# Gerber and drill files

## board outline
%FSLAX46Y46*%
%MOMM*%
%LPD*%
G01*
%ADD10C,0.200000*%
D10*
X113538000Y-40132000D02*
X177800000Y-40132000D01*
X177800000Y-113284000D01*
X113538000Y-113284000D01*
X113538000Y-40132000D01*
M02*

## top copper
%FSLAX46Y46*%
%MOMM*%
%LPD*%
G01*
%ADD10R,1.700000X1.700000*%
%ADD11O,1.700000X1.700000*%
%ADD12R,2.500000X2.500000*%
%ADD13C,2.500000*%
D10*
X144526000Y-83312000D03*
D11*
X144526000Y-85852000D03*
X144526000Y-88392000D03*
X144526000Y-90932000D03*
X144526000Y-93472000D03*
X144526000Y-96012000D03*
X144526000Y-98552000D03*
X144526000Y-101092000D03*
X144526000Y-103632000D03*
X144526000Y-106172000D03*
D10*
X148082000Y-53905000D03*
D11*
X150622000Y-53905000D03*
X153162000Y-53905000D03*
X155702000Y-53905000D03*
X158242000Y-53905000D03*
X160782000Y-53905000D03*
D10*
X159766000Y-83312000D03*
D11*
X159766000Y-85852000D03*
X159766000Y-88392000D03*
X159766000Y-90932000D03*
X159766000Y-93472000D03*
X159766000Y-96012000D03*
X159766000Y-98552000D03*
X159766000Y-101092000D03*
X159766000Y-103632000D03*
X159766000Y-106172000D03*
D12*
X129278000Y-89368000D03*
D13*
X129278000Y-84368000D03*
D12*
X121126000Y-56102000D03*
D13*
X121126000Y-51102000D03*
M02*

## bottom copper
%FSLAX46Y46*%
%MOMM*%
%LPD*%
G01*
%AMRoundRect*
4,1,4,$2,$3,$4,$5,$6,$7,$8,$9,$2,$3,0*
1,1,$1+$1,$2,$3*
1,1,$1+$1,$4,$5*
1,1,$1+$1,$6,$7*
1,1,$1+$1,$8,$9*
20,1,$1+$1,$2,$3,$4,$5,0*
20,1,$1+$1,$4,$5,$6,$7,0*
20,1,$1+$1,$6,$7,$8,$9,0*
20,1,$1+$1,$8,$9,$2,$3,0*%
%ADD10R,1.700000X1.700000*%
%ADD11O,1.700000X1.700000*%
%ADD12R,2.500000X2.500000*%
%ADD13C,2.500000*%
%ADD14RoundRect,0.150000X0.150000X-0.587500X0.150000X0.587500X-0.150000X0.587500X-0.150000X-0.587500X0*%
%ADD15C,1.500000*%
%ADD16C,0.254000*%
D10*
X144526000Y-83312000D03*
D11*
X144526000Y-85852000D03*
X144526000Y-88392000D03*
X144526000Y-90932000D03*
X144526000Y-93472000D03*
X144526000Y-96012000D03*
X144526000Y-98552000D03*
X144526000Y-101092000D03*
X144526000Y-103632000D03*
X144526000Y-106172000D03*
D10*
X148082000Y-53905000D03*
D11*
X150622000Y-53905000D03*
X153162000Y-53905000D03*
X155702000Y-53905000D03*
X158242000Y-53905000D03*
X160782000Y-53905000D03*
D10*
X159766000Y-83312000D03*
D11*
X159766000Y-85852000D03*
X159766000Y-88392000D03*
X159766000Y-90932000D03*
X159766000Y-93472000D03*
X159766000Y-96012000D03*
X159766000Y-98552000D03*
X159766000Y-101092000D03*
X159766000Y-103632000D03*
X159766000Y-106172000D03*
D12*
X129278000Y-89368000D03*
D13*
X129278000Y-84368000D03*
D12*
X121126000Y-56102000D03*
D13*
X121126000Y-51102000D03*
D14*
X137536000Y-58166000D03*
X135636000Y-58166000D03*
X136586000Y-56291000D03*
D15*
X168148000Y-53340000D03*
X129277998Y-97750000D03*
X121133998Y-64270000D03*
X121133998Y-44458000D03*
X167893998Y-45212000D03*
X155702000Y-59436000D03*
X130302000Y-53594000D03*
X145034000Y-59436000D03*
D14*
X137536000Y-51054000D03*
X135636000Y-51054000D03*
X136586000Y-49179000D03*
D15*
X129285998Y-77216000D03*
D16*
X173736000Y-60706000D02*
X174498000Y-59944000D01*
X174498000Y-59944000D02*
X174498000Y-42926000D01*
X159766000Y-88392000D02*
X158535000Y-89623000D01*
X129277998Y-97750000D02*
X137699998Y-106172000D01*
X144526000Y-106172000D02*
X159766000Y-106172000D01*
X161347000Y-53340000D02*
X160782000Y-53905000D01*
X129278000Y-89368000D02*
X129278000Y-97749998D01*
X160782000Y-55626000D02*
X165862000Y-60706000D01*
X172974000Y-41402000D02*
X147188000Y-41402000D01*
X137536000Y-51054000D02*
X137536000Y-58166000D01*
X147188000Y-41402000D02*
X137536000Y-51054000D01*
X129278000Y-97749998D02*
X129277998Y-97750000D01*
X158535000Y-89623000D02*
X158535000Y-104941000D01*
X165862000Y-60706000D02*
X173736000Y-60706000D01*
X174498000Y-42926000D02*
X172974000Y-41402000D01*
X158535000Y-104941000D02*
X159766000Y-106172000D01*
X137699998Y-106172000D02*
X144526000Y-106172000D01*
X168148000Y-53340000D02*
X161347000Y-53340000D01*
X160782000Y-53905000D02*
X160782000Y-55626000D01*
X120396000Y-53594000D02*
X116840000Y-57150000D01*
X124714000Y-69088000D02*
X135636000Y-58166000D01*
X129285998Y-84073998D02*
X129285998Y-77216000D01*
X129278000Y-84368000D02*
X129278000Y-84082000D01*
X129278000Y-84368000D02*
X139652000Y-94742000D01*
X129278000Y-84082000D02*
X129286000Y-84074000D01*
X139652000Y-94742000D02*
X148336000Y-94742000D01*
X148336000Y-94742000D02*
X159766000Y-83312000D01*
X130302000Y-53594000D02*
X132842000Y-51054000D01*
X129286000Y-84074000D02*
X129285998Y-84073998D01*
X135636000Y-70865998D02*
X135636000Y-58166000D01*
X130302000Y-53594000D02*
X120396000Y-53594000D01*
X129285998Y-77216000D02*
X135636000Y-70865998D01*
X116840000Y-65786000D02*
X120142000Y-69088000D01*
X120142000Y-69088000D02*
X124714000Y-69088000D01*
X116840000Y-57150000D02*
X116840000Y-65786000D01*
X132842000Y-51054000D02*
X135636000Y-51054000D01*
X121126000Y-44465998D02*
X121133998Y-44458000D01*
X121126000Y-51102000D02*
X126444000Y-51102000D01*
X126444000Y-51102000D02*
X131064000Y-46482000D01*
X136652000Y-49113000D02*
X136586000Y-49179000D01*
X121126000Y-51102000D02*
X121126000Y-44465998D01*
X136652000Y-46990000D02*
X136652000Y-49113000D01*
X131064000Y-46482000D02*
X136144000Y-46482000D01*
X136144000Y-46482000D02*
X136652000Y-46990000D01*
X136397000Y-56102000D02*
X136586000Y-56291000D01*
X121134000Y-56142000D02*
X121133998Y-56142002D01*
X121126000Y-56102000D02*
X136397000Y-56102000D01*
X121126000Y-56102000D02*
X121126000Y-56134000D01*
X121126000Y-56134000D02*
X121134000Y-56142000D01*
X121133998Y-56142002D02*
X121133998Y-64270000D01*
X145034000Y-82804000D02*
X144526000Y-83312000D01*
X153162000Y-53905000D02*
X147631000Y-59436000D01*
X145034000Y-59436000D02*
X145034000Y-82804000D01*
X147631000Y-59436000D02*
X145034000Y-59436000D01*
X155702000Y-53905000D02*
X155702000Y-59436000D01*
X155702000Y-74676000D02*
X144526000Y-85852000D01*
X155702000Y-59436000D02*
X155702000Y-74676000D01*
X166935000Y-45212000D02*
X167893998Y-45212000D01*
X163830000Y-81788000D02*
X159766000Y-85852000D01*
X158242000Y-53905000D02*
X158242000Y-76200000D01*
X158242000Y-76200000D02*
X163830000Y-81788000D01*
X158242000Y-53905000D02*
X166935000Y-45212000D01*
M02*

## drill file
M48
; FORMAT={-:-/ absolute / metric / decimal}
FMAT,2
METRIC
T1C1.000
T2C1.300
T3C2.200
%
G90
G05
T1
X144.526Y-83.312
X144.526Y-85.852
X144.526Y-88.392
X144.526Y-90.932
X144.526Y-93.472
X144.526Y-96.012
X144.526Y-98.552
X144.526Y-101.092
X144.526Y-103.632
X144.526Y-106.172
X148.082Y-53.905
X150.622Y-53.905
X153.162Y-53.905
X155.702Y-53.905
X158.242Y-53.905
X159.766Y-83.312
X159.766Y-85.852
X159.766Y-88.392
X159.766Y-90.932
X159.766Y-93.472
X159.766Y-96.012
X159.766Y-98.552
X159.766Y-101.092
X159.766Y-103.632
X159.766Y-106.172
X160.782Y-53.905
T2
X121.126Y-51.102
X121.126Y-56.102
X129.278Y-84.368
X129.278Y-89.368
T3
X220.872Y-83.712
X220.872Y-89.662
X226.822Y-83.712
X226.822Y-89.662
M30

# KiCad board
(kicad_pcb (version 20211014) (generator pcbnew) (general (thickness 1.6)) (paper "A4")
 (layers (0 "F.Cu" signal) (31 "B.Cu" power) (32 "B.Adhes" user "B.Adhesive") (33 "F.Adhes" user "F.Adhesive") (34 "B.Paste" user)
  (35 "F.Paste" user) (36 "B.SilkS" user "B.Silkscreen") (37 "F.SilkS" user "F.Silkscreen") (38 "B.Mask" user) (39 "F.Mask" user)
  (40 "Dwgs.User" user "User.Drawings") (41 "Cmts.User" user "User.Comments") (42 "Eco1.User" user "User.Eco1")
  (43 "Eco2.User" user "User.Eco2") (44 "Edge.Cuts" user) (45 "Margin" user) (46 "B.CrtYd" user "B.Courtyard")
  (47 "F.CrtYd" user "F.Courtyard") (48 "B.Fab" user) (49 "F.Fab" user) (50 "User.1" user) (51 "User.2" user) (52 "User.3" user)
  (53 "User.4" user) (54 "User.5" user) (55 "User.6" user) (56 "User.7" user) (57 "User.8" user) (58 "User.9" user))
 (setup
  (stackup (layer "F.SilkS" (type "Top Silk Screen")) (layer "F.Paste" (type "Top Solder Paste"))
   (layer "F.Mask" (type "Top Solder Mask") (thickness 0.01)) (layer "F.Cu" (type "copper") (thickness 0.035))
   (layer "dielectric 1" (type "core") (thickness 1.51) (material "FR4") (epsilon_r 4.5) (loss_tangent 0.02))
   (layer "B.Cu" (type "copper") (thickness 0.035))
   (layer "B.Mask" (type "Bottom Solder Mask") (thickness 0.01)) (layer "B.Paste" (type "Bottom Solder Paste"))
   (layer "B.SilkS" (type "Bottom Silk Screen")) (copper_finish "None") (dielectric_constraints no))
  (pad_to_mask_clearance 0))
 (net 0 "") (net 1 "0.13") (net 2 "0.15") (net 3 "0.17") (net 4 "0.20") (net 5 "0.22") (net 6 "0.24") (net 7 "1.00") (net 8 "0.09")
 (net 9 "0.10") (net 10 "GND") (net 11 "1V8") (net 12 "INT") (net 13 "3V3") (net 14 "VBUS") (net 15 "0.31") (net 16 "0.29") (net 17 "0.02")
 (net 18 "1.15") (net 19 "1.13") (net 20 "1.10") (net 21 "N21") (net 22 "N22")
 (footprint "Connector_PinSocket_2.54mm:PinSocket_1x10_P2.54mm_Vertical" (layer "F.Cu") (at 144.526 83.312)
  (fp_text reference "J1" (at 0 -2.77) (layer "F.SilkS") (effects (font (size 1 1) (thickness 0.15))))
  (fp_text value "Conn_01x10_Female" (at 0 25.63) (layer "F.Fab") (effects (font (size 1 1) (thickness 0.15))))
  (pad "1" thru_hole rect (at 0 0) (size 1.7 1.7) (drill 1) (layers *.Cu *.Mask) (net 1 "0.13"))
  (pad "2" thru_hole oval (at 0 2.54) (size 1.7 1.7) (drill 1) (layers *.Cu *.Mask) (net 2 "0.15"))
  (pad "3" thru_hole oval (at 0 5.08) (size 1.7 1.7) (drill 1) (layers *.Cu *.Mask) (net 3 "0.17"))
  (pad "4" thru_hole oval (at 0 7.62) (size 1.7 1.7) (drill 1) (layers *.Cu *.Mask) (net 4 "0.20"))
  (pad "5" thru_hole oval (at 0 10.16) (size 1.7 1.7) (drill 1) (layers *.Cu *.Mask) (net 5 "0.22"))
  (pad "6" thru_hole oval (at 0 12.7) (size 1.7 1.7) (drill 1) (layers *.Cu *.Mask) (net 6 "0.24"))
  (pad "7" thru_hole oval (at 0 15.24) (size 1.7 1.7) (drill 1) (layers *.Cu *.Mask) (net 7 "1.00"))
  (pad "8" thru_hole oval (at 0 17.78) (size 1.7 1.7) (drill 1) (layers *.Cu *.Mask) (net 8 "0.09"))
  (pad "9" thru_hole oval (at 0 20.32) (size 1.7 1.7) (drill 1) (layers *.Cu *.Mask) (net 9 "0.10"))
  (pad "10" thru_hole oval (at 0 22.86) (size 1.7 1.7) (drill 1) (layers *.Cu *.Mask) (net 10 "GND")))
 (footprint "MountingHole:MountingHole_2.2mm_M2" (layer "F.Cu") (at 226.822 83.712)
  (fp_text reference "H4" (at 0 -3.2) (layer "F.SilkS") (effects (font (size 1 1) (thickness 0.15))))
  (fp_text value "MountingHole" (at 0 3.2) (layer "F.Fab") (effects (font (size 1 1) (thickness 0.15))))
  (pad "" np_thru_hole circle (at 0 0) (size 2.2 2.2) (drill 2.2) (layers *.Cu *.Mask)))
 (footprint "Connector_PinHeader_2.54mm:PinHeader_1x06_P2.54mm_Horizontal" (layer "F.Cu") (at 148.082 53.905 90)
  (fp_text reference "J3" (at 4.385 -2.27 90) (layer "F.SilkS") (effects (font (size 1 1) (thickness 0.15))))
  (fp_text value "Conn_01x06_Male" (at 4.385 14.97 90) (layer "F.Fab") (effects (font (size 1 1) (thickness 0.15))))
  (pad "1" thru_hole rect (at 0 0 90) (size 1.7 1.7) (drill 1) (layers *.Cu *.Mask) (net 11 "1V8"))
  (pad "2" thru_hole oval (at 0 2.54 90) (size 1.7 1.7) (drill 1) (layers *.Cu *.Mask) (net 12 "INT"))
  (pad "3" thru_hole oval (at 0 5.08 90) (size 1.7 1.7) (drill 1) (layers *.Cu *.Mask) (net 1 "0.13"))
  (pad "4" thru_hole oval (at 0 7.62 90) (size 1.7 1.7) (drill 1) (layers *.Cu *.Mask) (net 2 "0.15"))
  (pad "5" thru_hole oval (at 0 10.16 90) (size 1.7 1.7) (drill 1) (layers *.Cu *.Mask) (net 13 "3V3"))
  (pad "6" thru_hole oval (at 0 12.7 90) (size 1.7 1.7) (drill 1) (layers *.Cu *.Mask) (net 10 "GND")))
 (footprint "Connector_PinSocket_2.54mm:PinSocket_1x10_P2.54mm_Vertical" (layer "F.Cu") (at 159.766 83.312)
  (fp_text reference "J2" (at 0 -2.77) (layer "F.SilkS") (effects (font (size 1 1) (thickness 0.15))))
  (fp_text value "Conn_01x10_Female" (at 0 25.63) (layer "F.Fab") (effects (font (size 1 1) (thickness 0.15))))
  (pad "1" thru_hole rect (at 0 0) (size 1.7 1.7) (drill 1) (layers *.Cu *.Mask) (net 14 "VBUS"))
  (pad "2" thru_hole oval (at 0 2.54) (size 1.7 1.7) (drill 1) (layers *.Cu *.Mask) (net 13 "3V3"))
  (pad "3" thru_hole oval (at 0 5.08) (size 1.7 1.7) (drill 1) (layers *.Cu *.Mask) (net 10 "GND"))
  (pad "4" thru_hole oval (at 0 7.62) (size 1.7 1.7) (drill 1) (layers *.Cu *.Mask) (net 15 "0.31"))
  (pad "5" thru_hole oval (at 0 10.16) (size 1.7 1.7) (drill 1) (layers *.Cu *.Mask) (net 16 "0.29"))
  (pad "6" thru_hole oval (at 0 12.7) (size 1.7 1.7) (drill 1) (layers *.Cu *.Mask) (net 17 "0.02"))
  (pad "7" thru_hole oval (at 0 15.24) (size 1.7 1.7) (drill 1) (layers *.Cu *.Mask) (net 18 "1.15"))
  (pad "8" thru_hole oval (at 0 17.78) (size 1.7 1.7) (drill 1) (layers *.Cu *.Mask) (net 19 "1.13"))
  (pad "9" thru_hole oval (at 0 20.32) (size 1.7 1.7) (drill 1) (layers *.Cu *.Mask) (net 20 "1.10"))
  (pad "10" thru_hole oval (at 0 22.86) (size 1.7 1.7) (drill 1) (layers *.Cu *.Mask) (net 10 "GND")))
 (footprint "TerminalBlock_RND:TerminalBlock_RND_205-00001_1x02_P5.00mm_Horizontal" (layer "F.Cu") (at 129.278 89.368 90)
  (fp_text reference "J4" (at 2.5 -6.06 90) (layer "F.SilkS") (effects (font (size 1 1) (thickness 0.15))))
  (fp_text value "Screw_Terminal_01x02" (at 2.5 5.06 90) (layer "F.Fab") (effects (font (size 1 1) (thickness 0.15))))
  (pad "1" thru_hole rect (at 0 0 90) (size 2.5 2.5) (drill 1.3) (layers *.Cu *.Mask) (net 10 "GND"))
  (pad "2" thru_hole circle (at 5 0 90) (size 2.5 2.5) (drill 1.3) (layers *.Cu *.Mask) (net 14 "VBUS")))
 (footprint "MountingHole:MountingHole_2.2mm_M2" (layer "F.Cu") (at 226.822 89.662)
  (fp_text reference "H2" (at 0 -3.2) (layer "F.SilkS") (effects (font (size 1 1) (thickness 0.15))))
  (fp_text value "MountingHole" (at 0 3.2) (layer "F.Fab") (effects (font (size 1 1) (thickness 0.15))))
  (pad "" np_thru_hole circle (at 0 0) (size 2.2 2.2) (drill 2.2) (layers *.Cu *.Mask)))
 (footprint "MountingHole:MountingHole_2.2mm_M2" (layer "F.Cu") (at 220.872 89.662)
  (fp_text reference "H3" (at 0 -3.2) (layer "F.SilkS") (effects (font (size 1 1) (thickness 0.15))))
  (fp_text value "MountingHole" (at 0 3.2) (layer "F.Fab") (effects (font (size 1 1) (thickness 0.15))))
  (pad "" np_thru_hole circle (at 0 0) (size 2.2 2.2) (drill 2.2) (layers *.Cu *.Mask)))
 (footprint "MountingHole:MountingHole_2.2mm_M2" (layer "F.Cu") (at 220.872 83.712)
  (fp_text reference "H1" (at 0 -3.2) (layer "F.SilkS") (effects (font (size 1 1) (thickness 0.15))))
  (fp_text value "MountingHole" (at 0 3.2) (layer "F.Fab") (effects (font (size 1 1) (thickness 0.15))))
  (pad "" np_thru_hole circle (at 0 0) (size 2.2 2.2) (drill 2.2) (layers *.Cu *.Mask)))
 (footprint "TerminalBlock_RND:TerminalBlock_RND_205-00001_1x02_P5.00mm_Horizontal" (layer "F.Cu") (at 121.126 56.102 90)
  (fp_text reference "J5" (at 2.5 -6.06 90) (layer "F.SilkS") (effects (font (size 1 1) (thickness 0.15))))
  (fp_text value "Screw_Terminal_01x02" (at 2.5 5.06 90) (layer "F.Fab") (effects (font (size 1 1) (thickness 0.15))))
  (pad "1" thru_hole rect (at 0 0 90) (size 2.5 2.5) (drill 1.3) (layers *.Cu *.Mask) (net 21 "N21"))
  (pad "2" thru_hole circle (at 5 0 90) (size 2.5 2.5) (drill 1.3) (layers *.Cu *.Mask) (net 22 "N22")))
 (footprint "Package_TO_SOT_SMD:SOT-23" (layer "B.Cu") (at 136.586 57.2285 90)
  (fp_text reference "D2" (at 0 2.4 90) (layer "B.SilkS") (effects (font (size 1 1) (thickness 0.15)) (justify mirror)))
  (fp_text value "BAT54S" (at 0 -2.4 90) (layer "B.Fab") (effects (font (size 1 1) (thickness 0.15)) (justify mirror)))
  (pad "1" smd roundrect (at -0.9375 0.95 90) (size 1.475 0.6) (layers "B.Cu" "B.Paste" "B.Mask") (roundrect_rratio 0.25) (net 10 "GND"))
  (pad "2" smd roundrect (at -0.9375 -0.95 90) (size 1.475 0.6) (layers "B.Cu" "B.Paste" "B.Mask") (roundrect_rratio 0.25) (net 14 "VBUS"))
  (pad "3" smd roundrect (at 0.9375 0 90) (size 1.475 0.6) (layers "B.Cu" "B.Paste" "B.Mask") (roundrect_rratio 0.25) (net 21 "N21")))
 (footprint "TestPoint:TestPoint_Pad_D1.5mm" (layer "B.Cu") (at 168.148 53.34 180)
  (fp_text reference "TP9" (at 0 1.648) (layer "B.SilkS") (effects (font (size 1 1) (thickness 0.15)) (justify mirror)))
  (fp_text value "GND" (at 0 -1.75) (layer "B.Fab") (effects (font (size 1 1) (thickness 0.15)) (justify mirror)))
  (pad "1" smd circle (at 0 0 180) (size 1.5 1.5) (layers "B.Cu" "B.Mask") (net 10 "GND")))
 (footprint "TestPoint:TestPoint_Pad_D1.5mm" (layer "B.Cu") (at 129.277998 97.75 90)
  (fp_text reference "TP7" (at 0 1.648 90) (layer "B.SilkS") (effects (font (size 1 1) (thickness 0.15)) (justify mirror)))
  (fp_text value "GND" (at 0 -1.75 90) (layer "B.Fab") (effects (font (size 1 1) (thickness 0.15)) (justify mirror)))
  (pad "1" smd circle (at 0 0 90) (size 1.5 1.5) (layers "B.Cu" "B.Mask") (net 10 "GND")))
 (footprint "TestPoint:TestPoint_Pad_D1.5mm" (layer "B.Cu") (at 121.133998 64.27 180)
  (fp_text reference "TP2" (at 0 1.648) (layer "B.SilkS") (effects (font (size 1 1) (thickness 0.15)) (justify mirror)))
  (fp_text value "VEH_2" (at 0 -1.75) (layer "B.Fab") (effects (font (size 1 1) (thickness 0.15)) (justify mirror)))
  (pad "1" smd circle (at 0 0 180) (size 1.5 1.5) (layers "B.Cu" "B.Mask") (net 21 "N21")))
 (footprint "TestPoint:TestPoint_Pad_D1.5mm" (layer "B.Cu") (at 121.133998 44.458 180)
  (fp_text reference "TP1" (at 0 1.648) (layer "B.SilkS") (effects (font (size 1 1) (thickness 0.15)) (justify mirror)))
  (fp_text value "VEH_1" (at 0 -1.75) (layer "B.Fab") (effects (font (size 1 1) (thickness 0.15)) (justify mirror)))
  (pad "1" smd circle (at 0 0 180) (size 1.5 1.5) (layers "B.Cu" "B.Mask") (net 22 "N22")))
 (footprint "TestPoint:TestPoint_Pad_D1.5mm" (layer "B.Cu") (at 167.893998 45.212 180)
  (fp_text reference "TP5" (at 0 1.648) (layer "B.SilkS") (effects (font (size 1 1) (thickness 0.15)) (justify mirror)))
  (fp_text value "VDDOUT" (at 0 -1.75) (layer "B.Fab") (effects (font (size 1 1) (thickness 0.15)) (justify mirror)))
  (pad "1" smd circle (at 0 0 180) (size 1.5 1.5) (layers "B.Cu" "B.Mask") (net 13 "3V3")))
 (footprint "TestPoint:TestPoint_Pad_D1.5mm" (layer "B.Cu") (at 155.702 59.436 180)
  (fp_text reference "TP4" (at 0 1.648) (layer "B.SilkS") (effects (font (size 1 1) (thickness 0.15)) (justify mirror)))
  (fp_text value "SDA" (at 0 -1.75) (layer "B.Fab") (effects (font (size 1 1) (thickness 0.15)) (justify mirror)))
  (pad "1" smd circle (at 0 0 180) (size 1.5 1.5) (layers "B.Cu" "B.Mask") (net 2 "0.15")))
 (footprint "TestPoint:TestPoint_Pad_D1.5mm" (layer "B.Cu") (at 130.302 53.594 180)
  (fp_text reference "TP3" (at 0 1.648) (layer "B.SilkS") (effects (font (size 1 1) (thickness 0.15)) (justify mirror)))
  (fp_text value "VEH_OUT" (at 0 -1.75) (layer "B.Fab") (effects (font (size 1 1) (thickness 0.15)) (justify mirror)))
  (pad "1" smd circle (at 0 0 180) (size 1.5 1.5) (layers "B.Cu" "B.Mask") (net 14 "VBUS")))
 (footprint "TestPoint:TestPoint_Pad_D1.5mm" (layer "B.Cu") (at 145.034 59.436 180)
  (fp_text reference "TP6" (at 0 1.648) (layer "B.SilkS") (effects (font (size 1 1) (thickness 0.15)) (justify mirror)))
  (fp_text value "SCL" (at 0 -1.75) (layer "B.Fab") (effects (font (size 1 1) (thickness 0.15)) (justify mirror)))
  (pad "1" smd circle (at 0 0 180) (size 1.5 1.5) (layers "B.Cu" "B.Mask") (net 1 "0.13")))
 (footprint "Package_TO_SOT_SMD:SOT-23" (layer "B.Cu") (at 136.586 50.1165 90)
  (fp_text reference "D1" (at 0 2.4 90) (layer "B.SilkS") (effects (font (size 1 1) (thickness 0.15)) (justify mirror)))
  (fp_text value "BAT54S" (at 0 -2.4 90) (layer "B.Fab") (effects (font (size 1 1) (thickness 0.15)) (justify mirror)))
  (pad "1" smd roundrect (at -0.9375 0.95 90) (size 1.475 0.6) (layers "B.Cu" "B.Paste" "B.Mask") (roundrect_rratio 0.25) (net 10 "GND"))
  (pad "2" smd roundrect (at -0.9375 -0.95 90) (size 1.475 0.6) (layers "B.Cu" "B.Paste" "B.Mask") (roundrect_rratio 0.25) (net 14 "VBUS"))
  (pad "3" smd roundrect (at 0.9375 0 90) (size 1.475 0.6) (layers "B.Cu" "B.Paste" "B.Mask") (roundrect_rratio 0.25) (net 22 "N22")))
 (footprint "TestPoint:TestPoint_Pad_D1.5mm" (layer "B.Cu") (at 129.285998 77.216 90)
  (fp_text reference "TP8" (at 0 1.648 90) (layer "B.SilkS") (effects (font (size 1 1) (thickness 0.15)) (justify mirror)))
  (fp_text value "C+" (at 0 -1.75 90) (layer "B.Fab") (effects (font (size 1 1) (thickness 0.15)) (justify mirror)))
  (pad "1" smd circle (at 0 0 90) (size 1.5 1.5) (layers "B.Cu" "B.Mask") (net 14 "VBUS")))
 (gr_rect (start 113.538 40.132) (end 177.8 113.284) (layer "Edge.Cuts") (width 0.2) (fill none))
 (segment (start 173.736 60.706) (end 174.498 59.944) (width 0.254) (layer "B.Cu") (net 10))
 (segment (start 174.498 59.944) (end 174.498 42.926) (width 0.254) (layer "B.Cu") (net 10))
 (segment (start 159.766 88.392) (end 158.535 89.623) (width 0.254) (layer "B.Cu") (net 10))
 (segment (start 129.277998 97.75) (end 137.699998 106.172) (width 0.254) (layer "B.Cu") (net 10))
 (segment (start 144.526 106.172) (end 159.766 106.172) (width 0.254) (layer "B.Cu") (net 10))
 (segment (start 161.347 53.34) (end 160.782 53.905) (width 0.254) (layer "B.Cu") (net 10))
 (segment (start 129.278 89.368) (end 129.278 97.749998) (width 0.254) (layer "B.Cu") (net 10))
 (segment (start 160.782 55.626) (end 165.862 60.706) (width 0.254) (layer "B.Cu") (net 10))
 (segment (start 172.974 41.402) (end 147.188 41.402) (width 0.254) (layer "B.Cu") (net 10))
 (segment (start 137.536 51.054) (end 137.536 58.166) (width 0.254) (layer "B.Cu") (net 10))
 (segment (start 147.188 41.402) (end 137.536 51.054) (width 0.254) (layer "B.Cu") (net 10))
 (segment (start 129.278 97.749998) (end 129.277998 97.75) (width 0.254) (layer "B.Cu") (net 10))
 (segment (start 158.535 89.623) (end 158.535 104.941) (width 0.254) (layer "B.Cu") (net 10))
 (segment (start 165.862 60.706) (end 173.736 60.706) (width 0.254) (layer "B.Cu") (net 10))
 (segment (start 174.498 42.926) (end 172.974 41.402) (width 0.254) (layer "B.Cu") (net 10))
 (segment (start 158.535 104.941) (end 159.766 106.172) (width 0.254) (layer "B.Cu") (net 10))
 (segment (start 137.699998 106.172) (end 144.526 106.172) (width 0.254) (layer "B.Cu") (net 10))
 (segment (start 168.148 53.34) (end 161.347 53.34) (width 0.254) (layer "B.Cu") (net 10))
 (segment (start 160.782 53.905) (end 160.782 55.626) (width 0.254) (layer "B.Cu") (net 10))
 (segment (start 120.396 53.594) (end 116.84 57.15) (width 0.254) (layer "B.Cu") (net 14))
 (segment (start 124.714 69.088) (end 135.636 58.166) (width 0.254) (layer "B.Cu") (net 14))
 (segment (start 129.285998 84.073998) (end 129.285998 77.216) (width 0.254) (layer "B.Cu") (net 14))
 (segment (start 129.278 84.368) (end 129.278 84.082) (width 0.254) (layer "B.Cu") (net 14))
 (segment (start 129.278 84.368) (end 139.652 94.742) (width 0.254) (layer "B.Cu") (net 14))
 (segment (start 129.278 84.082) (end 129.286 84.074) (width 0.254) (layer "B.Cu") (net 14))
 (segment (start 139.652 94.742) (end 148.336 94.742) (width 0.254) (layer "B.Cu") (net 14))
 (segment (start 148.336 94.742) (end 159.766 83.312) (width 0.254) (layer "B.Cu") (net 14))
 (segment (start 130.302 53.594) (end 132.842 51.054) (width 0.254) (layer "B.Cu") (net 14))
 (segment (start 129.286 84.074) (end 129.285998 84.073998) (width 0.254) (layer "B.Cu") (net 14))
 (segment (start 135.636 70.865998) (end 135.636 58.166) (width 0.254) (layer "B.Cu") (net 14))
 (segment (start 130.302 53.594) (end 120.396 53.594) (width 0.254) (layer "B.Cu") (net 14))
 (segment (start 129.285998 77.216) (end 135.636 70.865998) (width 0.254) (layer "B.Cu") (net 14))
 (segment (start 116.84 65.786) (end 120.142 69.088) (width 0.254) (layer "B.Cu") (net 14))
 (segment (start 120.142 69.088) (end 124.714 69.088) (width 0.254) (layer "B.Cu") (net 14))
 (segment (start 116.84 57.15) (end 116.84 65.786) (width 0.254) (layer "B.Cu") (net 14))
 (segment (start 132.842 51.054) (end 135.636 51.054) (width 0.254) (layer "B.Cu") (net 14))
 (segment (start 121.126 44.465998) (end 121.133998 44.458) (width 0.254) (layer "B.Cu") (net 22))
 (segment (start 121.126 51.102) (end 126.444 51.102) (width 0.254) (layer "B.Cu") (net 22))
 (segment (start 126.444 51.102) (end 131.064 46.482) (width 0.254) (layer "B.Cu") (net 22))
 (segment (start 136.652 49.113) (end 136.586 49.179) (width 0.254) (layer "B.Cu") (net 22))
 (segment (start 121.126 51.102) (end 121.126 44.465998) (width 0.254) (layer "B.Cu") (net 22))
 (segment (start 136.652 46.99) (end 136.652 49.113) (width 0.254) (layer "B.Cu") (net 22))
 (segment (start 131.064 46.482) (end 136.144 46.482) (width 0.254) (layer "B.Cu") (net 22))
 (segment (start 136.144 46.482) (end 136.652 46.99) (width 0.254) (layer "B.Cu") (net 22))
 (segment (start 136.397 56.102) (end 136.586 56.291) (width 0.254) (layer "B.Cu") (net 21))
 (segment (start 121.134 56.142) (end 121.133998 56.142002) (width 0.254) (layer "B.Cu") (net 21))
 (segment (start 121.126 56.102) (end 136.397 56.102) (width 0.254) (layer "B.Cu") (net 21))
 (segment (start 121.126 56.102) (end 121.126 56.134) (width 0.254) (layer "B.Cu") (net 21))
 (segment (start 121.126 56.134) (end 121.134 56.142) (width 0.254) (layer "B.Cu") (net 21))
 (segment (start 121.133998 56.142002) (end 121.133998 64.27) (width 0.254) (layer "B.Cu") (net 21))
 (segment (start 145.034 82.804) (end 144.526 83.312) (width 0.254) (layer "B.Cu") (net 1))
 (segment (start 153.162 53.905) (end 147.631 59.436) (width 0.254) (layer "B.Cu") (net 1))
 (segment (start 145.034 59.436) (end 145.034 82.804) (width 0.254) (layer "B.Cu") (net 1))
 (segment (start 147.631 59.436) (end 145.034 59.436) (width 0.254) (layer "B.Cu") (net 1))
 (segment (start 155.702 53.905) (end 155.702 59.436) (width 0.254) (layer "B.Cu") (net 2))
 (segment (start 155.702 74.676) (end 144.526 85.852) (width 0.254) (layer "B.Cu") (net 2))
 (segment (start 155.702 59.436) (end 155.702 74.676) (width 0.254) (layer "B.Cu") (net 2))
 (segment (start 166.935 45.212) (end 167.893998 45.212) (width 0.254) (layer "B.Cu") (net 13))
 (segment (start 163.83 81.788) (end 159.766 85.852) (width 0.254) (layer "B.Cu") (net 13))
 (segment (start 158.242 53.905) (end 158.242 76.2) (width 0.254) (layer "B.Cu") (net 13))
 (segment (start 158.242 76.2) (end 163.83 81.788) (width 0.254) (layer "B.Cu") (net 13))
 (segment (start 158.242 53.905) (end 166.935 45.212) (width 0.254) (layer "B.Cu") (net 13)))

